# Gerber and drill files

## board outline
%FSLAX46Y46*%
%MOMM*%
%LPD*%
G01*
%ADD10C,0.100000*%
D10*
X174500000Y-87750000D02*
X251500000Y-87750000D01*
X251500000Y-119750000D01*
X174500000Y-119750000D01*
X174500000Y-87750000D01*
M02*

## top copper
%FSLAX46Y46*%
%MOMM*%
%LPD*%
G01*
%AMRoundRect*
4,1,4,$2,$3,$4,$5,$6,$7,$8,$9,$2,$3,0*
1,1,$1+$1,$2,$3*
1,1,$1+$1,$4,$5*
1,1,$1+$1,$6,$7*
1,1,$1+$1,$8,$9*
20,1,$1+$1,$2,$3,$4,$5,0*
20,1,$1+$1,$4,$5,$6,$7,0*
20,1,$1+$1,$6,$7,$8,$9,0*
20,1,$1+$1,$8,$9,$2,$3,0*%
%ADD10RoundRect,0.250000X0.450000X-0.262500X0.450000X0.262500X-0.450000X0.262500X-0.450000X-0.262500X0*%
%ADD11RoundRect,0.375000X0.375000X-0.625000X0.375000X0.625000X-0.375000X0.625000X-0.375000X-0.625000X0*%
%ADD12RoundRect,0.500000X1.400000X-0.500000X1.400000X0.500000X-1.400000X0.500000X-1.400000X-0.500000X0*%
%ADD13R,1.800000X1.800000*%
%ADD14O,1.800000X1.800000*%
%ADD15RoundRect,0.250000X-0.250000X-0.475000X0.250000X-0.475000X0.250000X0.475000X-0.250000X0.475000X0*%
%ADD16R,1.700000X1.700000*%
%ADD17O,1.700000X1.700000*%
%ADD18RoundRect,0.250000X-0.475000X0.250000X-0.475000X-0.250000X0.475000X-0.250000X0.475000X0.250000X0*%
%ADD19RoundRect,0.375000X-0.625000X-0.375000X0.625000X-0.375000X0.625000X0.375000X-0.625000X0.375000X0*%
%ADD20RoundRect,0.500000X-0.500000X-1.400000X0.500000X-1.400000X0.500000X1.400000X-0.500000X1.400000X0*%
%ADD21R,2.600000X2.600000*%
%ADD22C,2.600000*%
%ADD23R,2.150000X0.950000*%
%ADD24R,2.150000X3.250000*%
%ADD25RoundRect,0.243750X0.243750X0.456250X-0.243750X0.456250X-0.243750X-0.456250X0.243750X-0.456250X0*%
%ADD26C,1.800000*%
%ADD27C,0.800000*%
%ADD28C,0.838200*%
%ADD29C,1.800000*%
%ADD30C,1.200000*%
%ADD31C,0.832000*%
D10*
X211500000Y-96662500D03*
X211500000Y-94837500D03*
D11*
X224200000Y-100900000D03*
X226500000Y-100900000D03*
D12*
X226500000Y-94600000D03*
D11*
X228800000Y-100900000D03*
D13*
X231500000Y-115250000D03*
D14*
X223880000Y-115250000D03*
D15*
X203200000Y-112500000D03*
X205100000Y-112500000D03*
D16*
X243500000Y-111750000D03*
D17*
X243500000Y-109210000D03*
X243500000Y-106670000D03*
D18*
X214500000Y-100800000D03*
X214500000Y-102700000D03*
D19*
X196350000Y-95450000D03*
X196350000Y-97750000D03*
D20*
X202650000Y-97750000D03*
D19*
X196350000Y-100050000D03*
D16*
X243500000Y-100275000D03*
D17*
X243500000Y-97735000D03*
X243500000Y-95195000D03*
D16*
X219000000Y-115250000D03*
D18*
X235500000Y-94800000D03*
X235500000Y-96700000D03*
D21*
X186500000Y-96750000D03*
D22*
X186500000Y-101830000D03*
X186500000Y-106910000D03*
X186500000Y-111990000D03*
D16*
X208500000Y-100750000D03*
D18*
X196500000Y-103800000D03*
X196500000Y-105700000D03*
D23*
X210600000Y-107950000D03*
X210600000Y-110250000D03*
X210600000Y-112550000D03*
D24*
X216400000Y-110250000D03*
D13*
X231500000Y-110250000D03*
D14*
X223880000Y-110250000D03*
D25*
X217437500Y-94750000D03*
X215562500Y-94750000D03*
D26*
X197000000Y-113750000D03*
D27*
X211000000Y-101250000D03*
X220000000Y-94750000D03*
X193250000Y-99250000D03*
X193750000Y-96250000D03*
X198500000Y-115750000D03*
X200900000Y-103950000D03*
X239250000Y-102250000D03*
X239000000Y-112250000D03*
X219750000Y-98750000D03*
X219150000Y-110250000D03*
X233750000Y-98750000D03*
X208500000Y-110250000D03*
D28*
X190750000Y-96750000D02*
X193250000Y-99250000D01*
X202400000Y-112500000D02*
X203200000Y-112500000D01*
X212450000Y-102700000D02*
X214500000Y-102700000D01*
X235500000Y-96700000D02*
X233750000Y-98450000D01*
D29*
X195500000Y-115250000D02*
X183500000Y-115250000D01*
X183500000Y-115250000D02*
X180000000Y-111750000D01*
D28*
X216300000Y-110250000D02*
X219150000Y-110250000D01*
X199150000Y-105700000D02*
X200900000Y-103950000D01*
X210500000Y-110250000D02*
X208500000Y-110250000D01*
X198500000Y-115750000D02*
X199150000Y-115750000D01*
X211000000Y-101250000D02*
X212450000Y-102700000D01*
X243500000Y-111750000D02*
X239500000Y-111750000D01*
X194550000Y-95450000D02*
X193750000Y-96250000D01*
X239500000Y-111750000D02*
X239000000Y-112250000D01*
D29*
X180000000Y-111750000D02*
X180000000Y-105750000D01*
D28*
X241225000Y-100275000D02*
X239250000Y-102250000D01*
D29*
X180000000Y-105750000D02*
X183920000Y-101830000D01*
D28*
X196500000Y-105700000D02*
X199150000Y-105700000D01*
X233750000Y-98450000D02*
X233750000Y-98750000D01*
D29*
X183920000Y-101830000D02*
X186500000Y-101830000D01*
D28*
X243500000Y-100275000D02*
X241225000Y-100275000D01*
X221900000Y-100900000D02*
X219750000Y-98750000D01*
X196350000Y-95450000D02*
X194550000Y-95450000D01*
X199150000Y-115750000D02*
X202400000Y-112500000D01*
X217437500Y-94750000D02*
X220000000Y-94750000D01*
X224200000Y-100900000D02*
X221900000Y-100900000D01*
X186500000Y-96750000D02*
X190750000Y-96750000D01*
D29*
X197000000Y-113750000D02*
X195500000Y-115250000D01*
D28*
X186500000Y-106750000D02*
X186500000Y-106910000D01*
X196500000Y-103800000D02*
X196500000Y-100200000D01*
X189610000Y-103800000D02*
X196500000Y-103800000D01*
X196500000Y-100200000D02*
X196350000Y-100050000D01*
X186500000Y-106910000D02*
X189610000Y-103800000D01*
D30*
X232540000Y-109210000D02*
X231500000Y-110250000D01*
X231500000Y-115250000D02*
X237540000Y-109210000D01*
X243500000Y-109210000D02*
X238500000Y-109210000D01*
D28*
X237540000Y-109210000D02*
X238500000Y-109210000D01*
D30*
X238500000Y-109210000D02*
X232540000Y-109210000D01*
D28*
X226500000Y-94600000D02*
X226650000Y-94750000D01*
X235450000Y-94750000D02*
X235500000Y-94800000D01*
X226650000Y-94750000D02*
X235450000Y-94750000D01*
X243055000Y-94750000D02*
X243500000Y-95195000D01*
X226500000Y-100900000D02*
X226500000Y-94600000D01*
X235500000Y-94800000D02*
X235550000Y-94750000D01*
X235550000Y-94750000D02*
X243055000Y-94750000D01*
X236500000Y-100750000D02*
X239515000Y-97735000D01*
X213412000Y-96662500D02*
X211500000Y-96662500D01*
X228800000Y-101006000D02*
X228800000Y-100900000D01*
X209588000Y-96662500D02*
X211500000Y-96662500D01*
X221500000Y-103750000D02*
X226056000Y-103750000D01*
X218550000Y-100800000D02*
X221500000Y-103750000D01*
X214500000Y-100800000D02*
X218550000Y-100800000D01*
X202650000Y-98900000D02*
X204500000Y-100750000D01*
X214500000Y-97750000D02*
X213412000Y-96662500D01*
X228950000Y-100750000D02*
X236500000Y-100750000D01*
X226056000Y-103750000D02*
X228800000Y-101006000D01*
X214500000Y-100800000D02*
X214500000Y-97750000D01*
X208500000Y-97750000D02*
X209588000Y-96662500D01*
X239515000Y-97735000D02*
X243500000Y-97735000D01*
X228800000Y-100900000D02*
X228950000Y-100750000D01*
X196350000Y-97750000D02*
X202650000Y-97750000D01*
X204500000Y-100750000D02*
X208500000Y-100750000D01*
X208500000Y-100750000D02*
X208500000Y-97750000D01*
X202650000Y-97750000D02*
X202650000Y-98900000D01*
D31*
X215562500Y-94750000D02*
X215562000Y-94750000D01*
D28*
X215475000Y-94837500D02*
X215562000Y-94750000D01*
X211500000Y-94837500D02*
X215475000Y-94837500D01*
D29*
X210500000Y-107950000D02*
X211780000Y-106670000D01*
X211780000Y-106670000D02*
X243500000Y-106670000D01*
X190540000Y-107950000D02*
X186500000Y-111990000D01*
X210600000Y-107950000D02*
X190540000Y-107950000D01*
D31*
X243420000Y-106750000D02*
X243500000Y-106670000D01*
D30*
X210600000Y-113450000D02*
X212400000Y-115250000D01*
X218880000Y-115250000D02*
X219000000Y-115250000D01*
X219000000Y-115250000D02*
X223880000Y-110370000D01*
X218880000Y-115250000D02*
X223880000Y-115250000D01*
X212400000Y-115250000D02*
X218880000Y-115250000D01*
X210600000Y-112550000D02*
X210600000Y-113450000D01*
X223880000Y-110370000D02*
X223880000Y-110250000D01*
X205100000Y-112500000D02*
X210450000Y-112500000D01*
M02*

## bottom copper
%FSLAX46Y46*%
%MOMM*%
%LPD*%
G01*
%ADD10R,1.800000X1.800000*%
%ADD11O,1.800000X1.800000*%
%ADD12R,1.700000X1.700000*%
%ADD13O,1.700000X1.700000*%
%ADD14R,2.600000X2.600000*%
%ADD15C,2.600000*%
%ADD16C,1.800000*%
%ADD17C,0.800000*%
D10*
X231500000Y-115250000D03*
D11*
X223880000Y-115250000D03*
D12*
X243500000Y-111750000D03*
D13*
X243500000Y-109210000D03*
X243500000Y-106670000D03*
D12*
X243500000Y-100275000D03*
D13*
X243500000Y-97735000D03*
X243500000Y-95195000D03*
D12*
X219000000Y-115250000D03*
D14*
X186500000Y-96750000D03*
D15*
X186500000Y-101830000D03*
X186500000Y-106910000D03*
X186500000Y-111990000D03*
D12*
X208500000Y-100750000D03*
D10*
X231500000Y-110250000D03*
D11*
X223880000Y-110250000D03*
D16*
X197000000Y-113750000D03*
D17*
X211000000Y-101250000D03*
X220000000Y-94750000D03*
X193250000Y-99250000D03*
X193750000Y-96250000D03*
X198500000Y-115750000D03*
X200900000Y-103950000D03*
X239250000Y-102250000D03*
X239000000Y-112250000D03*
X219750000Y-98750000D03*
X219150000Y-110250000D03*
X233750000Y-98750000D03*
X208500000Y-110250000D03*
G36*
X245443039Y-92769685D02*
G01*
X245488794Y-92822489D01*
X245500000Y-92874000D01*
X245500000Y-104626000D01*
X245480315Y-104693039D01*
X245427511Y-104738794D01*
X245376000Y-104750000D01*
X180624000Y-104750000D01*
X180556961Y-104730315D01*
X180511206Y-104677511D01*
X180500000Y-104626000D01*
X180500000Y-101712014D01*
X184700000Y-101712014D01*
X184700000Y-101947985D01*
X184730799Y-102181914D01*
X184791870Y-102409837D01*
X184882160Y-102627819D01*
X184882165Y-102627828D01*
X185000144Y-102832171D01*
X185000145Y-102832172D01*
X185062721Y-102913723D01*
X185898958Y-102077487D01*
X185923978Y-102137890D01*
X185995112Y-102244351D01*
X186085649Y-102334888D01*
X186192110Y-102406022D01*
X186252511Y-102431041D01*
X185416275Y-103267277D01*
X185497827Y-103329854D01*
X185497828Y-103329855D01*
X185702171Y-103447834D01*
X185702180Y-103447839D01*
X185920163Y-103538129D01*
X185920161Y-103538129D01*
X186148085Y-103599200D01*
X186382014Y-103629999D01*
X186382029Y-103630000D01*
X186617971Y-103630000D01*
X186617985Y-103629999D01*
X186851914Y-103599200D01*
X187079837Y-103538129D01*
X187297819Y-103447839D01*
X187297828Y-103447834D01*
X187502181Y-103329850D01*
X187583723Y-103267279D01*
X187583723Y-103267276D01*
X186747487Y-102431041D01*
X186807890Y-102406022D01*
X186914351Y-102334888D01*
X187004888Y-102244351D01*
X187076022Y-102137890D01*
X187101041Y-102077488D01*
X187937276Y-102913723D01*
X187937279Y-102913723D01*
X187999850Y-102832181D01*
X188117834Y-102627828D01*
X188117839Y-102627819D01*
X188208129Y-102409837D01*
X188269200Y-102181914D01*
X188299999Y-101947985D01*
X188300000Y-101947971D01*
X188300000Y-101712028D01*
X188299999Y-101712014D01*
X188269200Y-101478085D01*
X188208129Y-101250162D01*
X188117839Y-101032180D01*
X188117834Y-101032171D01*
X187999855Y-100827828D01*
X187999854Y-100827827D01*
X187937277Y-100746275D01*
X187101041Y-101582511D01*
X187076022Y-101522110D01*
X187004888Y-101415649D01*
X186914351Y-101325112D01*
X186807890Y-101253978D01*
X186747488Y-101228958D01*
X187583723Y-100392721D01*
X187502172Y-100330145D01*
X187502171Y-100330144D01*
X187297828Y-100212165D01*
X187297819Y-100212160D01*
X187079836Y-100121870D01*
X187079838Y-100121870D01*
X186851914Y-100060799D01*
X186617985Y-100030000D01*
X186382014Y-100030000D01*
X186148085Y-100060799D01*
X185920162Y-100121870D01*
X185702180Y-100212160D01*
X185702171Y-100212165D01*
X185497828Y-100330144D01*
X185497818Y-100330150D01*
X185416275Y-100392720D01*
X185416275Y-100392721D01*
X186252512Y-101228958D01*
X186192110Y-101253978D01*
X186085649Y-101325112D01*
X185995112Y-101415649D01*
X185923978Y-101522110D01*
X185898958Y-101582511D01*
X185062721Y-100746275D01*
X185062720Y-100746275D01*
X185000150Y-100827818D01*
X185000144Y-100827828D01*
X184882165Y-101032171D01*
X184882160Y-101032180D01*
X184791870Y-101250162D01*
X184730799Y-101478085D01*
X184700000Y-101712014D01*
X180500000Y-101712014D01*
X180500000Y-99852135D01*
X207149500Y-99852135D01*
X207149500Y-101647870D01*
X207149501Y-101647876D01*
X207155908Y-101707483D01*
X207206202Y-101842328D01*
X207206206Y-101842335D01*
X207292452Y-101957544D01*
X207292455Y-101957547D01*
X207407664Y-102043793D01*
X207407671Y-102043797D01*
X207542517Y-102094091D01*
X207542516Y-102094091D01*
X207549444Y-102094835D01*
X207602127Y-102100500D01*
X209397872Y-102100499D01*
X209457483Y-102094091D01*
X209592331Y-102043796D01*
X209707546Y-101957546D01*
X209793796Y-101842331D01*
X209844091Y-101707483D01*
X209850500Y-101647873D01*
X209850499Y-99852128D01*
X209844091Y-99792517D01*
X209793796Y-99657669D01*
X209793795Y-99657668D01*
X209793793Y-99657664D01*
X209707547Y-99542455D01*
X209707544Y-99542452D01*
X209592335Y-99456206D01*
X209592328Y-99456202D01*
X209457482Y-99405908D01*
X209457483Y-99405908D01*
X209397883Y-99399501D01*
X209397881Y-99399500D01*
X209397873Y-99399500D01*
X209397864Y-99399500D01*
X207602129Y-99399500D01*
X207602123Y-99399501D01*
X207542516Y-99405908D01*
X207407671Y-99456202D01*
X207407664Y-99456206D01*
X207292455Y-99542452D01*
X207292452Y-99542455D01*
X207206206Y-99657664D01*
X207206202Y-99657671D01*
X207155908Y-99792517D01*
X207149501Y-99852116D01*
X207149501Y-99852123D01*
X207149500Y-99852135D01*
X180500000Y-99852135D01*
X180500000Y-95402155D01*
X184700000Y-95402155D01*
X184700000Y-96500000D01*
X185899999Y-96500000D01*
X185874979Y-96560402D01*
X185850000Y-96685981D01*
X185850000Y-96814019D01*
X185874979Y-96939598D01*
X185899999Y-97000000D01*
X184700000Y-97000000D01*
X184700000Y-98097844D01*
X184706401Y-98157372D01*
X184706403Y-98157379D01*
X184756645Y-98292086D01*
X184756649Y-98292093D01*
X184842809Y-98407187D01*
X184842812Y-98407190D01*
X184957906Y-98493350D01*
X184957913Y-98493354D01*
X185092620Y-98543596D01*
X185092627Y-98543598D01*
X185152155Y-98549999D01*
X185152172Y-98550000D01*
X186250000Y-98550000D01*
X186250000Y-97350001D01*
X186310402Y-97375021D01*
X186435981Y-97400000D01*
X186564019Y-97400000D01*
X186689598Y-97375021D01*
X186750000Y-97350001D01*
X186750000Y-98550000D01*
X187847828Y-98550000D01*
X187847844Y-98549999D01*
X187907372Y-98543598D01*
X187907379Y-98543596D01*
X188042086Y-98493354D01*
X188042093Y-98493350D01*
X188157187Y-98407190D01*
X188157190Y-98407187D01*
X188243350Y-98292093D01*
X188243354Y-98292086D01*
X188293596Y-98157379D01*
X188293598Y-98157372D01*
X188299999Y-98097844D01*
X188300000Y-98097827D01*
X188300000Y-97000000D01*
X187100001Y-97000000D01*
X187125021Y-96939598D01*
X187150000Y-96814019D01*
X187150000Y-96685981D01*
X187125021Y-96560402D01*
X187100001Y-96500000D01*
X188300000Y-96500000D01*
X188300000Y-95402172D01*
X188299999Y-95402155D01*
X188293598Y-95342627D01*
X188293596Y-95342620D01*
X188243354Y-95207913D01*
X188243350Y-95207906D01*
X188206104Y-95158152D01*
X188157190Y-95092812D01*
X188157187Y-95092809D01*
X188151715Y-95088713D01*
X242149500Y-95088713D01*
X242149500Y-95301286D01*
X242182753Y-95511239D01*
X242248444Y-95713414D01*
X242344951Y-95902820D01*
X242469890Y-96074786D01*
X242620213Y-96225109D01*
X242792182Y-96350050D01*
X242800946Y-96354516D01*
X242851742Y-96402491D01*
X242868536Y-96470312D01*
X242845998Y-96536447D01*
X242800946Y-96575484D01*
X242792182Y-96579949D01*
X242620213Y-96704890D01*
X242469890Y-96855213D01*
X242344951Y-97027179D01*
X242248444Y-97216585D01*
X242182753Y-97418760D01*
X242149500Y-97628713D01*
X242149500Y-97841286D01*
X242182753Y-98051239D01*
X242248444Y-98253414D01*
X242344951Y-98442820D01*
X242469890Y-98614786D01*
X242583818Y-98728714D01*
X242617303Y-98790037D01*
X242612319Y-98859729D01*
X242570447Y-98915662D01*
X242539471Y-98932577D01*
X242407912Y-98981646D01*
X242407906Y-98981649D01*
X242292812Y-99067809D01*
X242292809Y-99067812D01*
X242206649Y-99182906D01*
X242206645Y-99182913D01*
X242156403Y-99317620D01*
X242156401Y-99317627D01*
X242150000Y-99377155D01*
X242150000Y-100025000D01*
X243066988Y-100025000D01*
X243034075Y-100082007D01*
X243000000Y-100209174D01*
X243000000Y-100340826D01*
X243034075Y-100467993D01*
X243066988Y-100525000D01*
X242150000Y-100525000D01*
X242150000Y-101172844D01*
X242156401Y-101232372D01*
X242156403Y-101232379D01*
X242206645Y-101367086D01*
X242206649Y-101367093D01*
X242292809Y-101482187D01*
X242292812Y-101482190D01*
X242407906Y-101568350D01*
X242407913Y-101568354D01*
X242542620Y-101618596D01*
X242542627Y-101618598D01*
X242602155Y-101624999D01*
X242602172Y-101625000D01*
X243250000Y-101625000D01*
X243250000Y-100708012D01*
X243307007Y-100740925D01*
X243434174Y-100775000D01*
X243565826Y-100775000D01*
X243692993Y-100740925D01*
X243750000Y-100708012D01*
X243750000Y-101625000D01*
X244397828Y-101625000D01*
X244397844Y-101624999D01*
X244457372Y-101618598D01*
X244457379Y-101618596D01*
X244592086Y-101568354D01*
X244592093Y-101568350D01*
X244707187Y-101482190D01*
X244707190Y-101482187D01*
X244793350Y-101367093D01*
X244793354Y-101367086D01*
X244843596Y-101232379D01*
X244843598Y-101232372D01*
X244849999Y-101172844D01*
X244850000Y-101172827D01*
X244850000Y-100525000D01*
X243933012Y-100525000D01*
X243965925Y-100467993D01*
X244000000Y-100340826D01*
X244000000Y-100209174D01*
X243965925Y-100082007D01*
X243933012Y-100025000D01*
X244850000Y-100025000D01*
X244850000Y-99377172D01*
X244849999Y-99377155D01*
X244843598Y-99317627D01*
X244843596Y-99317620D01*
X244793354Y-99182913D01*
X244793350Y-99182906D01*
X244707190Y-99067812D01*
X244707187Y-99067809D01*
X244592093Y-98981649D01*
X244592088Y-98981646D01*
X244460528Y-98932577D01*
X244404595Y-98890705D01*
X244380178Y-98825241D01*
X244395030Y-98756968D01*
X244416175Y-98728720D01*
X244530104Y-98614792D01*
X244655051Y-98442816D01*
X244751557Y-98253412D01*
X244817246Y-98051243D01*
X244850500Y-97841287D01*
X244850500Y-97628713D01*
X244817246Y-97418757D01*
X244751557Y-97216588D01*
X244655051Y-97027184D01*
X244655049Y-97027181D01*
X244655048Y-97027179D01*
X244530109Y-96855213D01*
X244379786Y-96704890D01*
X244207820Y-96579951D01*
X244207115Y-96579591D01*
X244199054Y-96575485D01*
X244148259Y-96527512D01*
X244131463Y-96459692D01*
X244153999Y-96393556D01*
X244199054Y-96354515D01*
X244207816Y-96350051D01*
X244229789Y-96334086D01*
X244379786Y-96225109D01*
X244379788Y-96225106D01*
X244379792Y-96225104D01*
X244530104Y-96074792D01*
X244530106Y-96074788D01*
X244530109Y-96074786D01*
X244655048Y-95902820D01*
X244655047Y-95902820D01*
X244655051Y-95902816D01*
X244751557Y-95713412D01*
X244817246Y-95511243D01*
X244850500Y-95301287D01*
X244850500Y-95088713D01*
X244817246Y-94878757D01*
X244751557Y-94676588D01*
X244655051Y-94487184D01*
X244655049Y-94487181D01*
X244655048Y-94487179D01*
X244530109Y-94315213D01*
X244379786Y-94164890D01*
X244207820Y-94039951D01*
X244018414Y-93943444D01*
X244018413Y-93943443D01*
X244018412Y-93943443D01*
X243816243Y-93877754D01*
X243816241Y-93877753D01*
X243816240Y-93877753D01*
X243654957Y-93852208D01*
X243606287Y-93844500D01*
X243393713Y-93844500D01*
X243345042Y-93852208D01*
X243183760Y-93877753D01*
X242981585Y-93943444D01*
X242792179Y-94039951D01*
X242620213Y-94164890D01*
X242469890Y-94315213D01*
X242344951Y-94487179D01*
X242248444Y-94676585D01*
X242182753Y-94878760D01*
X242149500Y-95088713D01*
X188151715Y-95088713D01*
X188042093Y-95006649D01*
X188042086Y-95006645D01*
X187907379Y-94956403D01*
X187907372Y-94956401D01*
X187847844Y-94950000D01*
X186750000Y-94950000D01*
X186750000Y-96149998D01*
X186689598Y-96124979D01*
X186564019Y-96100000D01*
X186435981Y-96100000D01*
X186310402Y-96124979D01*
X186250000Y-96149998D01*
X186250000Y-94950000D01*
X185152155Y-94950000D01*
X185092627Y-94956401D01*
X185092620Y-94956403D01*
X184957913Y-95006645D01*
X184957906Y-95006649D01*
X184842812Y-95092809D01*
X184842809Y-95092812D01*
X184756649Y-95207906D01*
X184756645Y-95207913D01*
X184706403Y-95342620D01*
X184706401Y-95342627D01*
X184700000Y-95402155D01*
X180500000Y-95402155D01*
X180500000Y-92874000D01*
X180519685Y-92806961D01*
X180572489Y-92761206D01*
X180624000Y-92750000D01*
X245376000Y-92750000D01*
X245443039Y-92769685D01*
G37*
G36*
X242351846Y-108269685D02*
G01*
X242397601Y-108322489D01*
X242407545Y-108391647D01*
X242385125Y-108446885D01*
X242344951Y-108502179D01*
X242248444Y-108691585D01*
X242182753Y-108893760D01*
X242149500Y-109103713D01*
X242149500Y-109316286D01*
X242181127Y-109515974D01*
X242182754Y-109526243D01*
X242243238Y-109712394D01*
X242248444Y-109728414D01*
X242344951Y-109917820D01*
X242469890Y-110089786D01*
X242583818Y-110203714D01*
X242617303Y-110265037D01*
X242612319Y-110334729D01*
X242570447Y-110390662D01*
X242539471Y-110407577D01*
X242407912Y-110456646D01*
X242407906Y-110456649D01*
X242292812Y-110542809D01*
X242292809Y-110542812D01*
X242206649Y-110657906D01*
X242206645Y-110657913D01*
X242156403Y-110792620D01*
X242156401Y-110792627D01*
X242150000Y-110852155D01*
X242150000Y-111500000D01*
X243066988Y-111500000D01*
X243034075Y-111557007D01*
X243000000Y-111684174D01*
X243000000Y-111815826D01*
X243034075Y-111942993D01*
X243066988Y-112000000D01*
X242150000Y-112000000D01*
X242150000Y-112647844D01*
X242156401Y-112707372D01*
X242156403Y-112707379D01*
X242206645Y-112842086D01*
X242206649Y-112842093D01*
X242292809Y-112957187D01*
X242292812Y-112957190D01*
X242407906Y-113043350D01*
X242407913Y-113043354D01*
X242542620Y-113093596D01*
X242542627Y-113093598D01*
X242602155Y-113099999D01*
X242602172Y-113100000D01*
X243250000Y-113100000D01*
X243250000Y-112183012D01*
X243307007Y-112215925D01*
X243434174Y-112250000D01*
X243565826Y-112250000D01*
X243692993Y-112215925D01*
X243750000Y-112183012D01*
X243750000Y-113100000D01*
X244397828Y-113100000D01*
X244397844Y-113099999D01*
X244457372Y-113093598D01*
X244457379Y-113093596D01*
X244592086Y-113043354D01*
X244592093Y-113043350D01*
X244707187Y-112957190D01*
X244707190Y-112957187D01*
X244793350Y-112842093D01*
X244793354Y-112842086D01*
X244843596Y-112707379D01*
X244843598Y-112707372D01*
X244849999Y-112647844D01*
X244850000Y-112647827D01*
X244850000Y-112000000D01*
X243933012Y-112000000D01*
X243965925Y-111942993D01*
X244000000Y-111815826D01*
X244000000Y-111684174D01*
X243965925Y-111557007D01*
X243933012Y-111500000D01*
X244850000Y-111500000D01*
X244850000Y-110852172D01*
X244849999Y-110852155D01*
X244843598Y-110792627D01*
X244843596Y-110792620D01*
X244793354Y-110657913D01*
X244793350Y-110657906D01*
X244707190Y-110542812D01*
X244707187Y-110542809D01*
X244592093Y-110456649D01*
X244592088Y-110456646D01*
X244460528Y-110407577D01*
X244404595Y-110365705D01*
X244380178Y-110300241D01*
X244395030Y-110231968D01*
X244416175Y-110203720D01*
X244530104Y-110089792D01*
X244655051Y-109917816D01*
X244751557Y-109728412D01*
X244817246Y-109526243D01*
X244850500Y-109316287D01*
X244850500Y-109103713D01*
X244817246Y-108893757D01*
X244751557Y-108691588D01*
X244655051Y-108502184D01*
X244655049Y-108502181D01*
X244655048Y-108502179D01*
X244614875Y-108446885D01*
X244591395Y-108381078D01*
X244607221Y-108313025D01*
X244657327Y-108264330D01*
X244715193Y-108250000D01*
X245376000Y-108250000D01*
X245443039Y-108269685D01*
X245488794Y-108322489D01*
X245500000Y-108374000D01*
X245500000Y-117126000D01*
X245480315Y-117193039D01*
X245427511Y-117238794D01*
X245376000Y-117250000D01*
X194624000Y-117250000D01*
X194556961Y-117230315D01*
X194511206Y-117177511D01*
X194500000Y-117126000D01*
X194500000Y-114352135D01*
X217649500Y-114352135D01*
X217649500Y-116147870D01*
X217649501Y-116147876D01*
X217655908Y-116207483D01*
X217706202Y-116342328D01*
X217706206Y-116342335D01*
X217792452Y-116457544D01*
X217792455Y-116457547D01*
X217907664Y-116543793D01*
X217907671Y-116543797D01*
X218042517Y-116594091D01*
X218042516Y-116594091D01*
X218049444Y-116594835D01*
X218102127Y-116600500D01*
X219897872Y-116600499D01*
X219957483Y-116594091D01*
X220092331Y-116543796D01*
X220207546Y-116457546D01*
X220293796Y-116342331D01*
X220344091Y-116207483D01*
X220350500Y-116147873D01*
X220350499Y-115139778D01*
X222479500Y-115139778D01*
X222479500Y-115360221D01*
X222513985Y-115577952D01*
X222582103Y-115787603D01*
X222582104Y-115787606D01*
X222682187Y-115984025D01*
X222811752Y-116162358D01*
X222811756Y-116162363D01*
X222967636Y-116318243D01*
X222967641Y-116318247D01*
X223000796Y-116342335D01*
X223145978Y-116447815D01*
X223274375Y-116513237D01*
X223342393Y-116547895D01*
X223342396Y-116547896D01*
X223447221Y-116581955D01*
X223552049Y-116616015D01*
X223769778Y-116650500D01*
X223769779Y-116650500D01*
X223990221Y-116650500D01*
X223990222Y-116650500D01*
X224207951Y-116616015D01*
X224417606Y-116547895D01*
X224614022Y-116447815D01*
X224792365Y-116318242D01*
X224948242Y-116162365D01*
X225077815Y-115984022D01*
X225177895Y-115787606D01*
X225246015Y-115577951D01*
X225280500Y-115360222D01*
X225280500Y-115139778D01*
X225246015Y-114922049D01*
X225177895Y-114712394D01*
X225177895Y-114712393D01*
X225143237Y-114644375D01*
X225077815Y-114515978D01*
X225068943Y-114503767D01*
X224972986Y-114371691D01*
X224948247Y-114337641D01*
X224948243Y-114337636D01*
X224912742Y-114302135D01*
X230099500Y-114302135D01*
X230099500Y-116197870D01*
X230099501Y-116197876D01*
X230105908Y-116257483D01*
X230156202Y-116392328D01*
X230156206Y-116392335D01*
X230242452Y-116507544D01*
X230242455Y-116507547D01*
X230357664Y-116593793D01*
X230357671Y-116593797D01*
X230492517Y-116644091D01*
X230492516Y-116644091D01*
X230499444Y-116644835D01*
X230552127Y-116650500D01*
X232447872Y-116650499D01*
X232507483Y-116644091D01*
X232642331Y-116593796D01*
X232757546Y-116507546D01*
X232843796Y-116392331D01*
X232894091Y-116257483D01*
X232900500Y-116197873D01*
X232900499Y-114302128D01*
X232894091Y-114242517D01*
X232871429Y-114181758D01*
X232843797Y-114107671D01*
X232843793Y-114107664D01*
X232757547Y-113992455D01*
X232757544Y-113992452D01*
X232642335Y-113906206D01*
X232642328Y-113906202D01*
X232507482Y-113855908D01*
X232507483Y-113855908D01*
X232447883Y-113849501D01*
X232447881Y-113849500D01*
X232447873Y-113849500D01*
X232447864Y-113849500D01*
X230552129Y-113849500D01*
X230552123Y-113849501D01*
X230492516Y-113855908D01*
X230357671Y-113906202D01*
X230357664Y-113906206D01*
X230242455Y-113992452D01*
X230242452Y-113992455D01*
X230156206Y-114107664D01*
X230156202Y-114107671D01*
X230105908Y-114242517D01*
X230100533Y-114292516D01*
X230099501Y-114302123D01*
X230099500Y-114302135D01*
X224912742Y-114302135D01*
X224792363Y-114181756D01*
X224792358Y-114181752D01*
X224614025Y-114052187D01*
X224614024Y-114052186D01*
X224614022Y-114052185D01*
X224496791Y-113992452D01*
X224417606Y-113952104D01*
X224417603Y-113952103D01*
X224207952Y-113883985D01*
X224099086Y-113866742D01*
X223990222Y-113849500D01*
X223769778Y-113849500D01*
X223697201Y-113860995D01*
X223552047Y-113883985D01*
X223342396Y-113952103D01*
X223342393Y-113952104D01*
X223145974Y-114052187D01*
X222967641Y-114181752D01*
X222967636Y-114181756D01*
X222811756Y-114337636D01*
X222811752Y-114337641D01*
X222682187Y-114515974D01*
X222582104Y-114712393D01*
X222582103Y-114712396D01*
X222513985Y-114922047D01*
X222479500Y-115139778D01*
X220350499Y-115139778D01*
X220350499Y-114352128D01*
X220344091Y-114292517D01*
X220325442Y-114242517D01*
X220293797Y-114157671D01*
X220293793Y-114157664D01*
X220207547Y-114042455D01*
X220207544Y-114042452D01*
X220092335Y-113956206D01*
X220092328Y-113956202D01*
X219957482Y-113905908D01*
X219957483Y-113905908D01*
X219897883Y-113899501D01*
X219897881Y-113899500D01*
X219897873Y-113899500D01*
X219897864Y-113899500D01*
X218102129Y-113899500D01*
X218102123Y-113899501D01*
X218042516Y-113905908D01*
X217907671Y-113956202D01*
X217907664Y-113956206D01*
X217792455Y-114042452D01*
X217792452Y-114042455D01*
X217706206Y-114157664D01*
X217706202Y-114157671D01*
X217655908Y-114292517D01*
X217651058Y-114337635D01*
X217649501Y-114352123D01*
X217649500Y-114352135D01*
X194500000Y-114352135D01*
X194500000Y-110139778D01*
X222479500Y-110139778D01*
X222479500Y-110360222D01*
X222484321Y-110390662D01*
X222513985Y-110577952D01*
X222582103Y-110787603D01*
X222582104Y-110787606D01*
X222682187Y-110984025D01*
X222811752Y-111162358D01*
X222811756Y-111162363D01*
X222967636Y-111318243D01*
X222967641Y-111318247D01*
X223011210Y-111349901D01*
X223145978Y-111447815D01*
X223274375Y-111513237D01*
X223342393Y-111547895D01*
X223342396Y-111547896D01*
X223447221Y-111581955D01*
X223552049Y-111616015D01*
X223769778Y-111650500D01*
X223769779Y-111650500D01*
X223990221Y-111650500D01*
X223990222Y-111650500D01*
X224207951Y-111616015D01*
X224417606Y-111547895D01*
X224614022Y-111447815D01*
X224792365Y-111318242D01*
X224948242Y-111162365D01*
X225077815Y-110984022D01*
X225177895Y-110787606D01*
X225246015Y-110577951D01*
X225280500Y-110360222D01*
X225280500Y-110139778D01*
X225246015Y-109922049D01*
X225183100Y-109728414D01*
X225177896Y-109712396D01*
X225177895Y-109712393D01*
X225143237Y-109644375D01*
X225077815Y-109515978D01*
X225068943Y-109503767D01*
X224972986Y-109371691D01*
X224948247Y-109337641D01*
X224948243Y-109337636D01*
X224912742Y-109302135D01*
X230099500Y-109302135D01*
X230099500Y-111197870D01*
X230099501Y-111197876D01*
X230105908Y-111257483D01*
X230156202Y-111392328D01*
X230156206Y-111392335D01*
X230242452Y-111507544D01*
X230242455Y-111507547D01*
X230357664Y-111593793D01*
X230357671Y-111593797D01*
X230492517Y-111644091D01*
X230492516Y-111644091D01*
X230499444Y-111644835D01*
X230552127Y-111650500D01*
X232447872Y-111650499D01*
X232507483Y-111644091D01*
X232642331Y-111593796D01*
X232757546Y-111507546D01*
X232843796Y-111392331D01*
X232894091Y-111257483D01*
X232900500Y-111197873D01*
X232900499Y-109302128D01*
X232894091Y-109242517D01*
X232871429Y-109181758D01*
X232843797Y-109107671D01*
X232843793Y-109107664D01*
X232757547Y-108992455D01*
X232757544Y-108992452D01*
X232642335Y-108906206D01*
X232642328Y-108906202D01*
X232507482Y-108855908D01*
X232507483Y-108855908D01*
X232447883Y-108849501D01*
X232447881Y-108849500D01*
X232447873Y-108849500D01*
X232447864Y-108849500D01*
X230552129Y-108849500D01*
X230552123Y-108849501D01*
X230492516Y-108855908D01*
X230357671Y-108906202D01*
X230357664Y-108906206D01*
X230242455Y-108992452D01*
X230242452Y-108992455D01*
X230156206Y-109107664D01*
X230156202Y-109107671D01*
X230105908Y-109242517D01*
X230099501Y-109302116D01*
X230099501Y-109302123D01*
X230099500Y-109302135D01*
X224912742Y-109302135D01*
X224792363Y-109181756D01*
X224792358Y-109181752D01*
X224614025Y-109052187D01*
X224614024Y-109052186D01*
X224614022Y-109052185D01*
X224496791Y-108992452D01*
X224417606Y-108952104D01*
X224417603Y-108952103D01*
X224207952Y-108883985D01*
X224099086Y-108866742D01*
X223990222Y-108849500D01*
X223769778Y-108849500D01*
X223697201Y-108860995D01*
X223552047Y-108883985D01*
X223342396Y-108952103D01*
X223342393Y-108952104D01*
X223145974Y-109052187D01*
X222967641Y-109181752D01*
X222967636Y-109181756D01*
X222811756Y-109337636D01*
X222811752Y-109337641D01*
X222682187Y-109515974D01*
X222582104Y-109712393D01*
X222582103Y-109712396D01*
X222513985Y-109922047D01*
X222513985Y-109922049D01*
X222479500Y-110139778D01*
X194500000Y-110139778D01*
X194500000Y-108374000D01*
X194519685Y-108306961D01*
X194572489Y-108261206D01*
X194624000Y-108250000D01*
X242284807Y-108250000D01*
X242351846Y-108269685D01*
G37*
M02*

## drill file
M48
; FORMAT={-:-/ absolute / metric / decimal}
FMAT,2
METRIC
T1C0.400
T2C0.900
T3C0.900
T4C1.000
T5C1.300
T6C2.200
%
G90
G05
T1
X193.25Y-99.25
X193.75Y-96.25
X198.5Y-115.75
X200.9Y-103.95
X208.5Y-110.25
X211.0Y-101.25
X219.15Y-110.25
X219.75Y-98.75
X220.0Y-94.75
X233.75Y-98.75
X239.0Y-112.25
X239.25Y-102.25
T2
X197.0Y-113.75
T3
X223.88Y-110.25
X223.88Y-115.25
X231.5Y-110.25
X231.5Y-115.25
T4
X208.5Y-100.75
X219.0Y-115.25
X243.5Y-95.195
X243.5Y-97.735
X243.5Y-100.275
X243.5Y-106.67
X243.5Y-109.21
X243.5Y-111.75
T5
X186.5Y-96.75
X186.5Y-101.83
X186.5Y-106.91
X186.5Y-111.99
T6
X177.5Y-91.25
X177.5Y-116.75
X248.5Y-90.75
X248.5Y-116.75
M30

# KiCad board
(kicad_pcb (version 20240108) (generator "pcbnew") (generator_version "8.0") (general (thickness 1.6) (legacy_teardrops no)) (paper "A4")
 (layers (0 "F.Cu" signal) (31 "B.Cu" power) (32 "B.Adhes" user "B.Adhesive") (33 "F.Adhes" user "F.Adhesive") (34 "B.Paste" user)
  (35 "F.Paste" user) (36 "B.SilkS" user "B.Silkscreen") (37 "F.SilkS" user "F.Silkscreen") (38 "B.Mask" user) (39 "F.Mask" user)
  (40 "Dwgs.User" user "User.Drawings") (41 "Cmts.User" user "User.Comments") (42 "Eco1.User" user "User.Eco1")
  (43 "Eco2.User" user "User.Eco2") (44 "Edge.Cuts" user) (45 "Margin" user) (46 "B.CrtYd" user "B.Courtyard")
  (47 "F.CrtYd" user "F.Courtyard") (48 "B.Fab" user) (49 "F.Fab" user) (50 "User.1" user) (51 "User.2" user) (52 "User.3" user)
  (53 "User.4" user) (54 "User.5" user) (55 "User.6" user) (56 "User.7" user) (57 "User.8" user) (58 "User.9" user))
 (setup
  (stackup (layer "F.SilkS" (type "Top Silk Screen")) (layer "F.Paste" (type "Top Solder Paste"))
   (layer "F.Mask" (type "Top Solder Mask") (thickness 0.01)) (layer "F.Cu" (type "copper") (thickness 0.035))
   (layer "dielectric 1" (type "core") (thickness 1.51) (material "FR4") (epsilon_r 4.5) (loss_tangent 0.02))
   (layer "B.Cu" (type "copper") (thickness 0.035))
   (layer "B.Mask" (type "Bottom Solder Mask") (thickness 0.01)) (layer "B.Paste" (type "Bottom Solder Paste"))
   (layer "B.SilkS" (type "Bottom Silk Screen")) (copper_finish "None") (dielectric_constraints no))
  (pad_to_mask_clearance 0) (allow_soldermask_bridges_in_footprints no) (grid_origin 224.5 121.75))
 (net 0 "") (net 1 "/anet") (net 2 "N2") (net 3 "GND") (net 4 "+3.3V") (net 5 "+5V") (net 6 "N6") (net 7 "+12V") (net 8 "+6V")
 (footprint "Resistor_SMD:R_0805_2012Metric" (layer "F.Cu") (at 211.5 95.75 90)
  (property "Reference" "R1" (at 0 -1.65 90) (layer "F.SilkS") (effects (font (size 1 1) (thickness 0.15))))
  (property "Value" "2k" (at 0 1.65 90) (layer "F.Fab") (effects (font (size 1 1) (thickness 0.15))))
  (pad "1" smd roundrect (at -0.9125 0 90) (size 1.025 1.4) (layers "F.Cu" "F.Paste" "F.Mask") (roundrect_rratio 0.243902) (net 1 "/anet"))
  (pad "2" smd roundrect (at 0.9125 0 90) (size 1.025 1.4) (layers "F.Cu" "F.Paste" "F.Mask") (roundrect_rratio 0.243902) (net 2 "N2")))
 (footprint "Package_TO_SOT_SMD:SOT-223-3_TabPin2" (layer "F.Cu") (at 226.5 97.75 90)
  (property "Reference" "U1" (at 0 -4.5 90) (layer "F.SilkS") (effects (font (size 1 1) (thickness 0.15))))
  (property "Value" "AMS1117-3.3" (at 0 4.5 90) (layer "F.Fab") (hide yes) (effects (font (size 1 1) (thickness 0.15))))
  (pad "1" smd roundrect (at -3.15 -2.3 90) (size 2 1.5) (layers "F.Cu" "F.Paste" "F.Mask") (roundrect_rratio 0.25) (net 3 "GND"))
  (pad "2" smd roundrect (at -3.15 0 90) (size 2 1.5) (layers "F.Cu" "F.Paste" "F.Mask") (roundrect_rratio 0.25) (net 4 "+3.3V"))
  (pad "2" smd roundrect (at 3.15 0 90) (size 2 3.8) (layers "F.Cu" "F.Paste" "F.Mask") (roundrect_rratio 0.25) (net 4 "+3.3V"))
  (pad "3" smd roundrect (at -3.15 2.3 90) (size 2 1.5) (layers "F.Cu" "F.Paste" "F.Mask") (roundrect_rratio 0.25) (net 1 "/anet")))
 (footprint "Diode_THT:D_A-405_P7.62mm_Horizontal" (layer "F.Cu") (at 231.5 115.25 180)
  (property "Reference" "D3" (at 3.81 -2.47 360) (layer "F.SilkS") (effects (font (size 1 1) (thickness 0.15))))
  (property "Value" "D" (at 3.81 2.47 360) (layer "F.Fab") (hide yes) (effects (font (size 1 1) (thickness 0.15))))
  (pad "1" thru_hole rect (at 0 0 180) (size 1.8 1.8) (drill 0.9) (layers "*.Cu" "*.Mask") (remove_unused_layers no) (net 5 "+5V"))
  (pad "2" thru_hole oval (at 7.62 0 180) (size 1.8 1.8) (drill 0.9) (layers "*.Cu" "*.Mask") (remove_unused_layers no) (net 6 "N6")))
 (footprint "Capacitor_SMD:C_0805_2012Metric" (layer "F.Cu") (at 204.15 112.5)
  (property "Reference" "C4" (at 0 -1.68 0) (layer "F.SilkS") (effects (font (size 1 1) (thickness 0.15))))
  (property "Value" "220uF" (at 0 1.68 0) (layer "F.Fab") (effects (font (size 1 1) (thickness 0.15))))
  (pad "1" smd roundrect (at -0.95 0) (size 1 1.45) (layers "F.Cu" "F.Paste" "F.Mask") (roundrect_rratio 0.25) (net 3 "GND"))
  (pad "2" smd roundrect (at 0.95 0) (size 1 1.45) (layers "F.Cu" "F.Paste" "F.Mask") (roundrect_rratio 0.25) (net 6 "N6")))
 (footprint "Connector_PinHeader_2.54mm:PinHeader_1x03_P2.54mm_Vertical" (layer "F.Cu") (at 243.5 111.75 180)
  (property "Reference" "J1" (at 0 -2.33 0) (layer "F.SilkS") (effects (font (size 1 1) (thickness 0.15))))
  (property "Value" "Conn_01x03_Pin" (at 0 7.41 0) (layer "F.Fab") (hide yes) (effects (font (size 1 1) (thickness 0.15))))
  (pad "1" thru_hole rect (at 0 0 180) (size 1.7 1.7) (drill 1) (layers "*.Cu" "*.Mask") (remove_unused_layers no) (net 3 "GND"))
  (pad "2" thru_hole oval (at 0 2.54 180) (size 1.7 1.7) (drill 1) (layers "*.Cu" "*.Mask") (remove_unused_layers no) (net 5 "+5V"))
  (pad "3" thru_hole oval (at 0 5.08 180) (size 1.7 1.7) (drill 1) (layers "*.Cu" "*.Mask") (remove_unused_layers no) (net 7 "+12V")))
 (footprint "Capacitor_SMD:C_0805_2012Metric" (layer "F.Cu") (at 214.5 101.75 -90)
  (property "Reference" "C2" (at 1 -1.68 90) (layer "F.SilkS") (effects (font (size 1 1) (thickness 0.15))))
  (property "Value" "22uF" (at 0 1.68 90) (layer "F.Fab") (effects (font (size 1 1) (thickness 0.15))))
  (pad "1" smd roundrect (at -0.95 0 270) (size 1 1.45) (layers "F.Cu" "F.Paste" "F.Mask") (roundrect_rratio 0.25) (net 1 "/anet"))
  (pad "2" smd roundrect (at 0.95 0 270) (size 1 1.45) (layers "F.Cu" "F.Paste" "F.Mask") (roundrect_rratio 0.25) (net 3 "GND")))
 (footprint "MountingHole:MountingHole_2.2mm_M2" (layer "F.Cu") (at 177.5 116.75)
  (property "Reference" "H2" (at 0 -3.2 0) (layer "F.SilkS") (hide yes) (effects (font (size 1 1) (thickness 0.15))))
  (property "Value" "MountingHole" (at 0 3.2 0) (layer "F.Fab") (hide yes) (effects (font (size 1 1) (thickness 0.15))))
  (pad "" np_thru_hole circle (at 0 0) (size 2.2 2.2) (drill 2.2) (layers "*.Cu" "*.Mask")))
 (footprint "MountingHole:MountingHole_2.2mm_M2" (layer "F.Cu") (at 177.5 91.25)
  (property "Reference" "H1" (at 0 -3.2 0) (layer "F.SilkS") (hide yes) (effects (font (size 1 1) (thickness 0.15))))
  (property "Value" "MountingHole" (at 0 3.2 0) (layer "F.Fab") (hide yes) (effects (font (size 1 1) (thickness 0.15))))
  (pad "" np_thru_hole circle (at 0 0) (size 2.2 2.2) (drill 2.2) (layers "*.Cu" "*.Mask")))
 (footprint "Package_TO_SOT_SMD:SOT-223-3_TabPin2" (layer "F.Cu") (at 199.5 97.75)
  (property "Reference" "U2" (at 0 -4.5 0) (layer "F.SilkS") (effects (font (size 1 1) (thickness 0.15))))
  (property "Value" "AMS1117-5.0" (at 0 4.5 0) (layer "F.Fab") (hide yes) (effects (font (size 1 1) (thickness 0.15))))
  (pad "1" smd roundrect (at -3.15 -2.3) (size 2 1.5) (layers "F.Cu" "F.Paste" "F.Mask") (roundrect_rratio 0.25) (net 3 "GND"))
  (pad "2" smd roundrect (at -3.15 0) (size 2 1.5) (layers "F.Cu" "F.Paste" "F.Mask") (roundrect_rratio 0.25) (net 1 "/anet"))
  (pad "2" smd roundrect (at 3.15 0) (size 2 3.8) (layers "F.Cu" "F.Paste" "F.Mask") (roundrect_rratio 0.25) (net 1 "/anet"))
  (pad "3" smd roundrect (at -3.15 2.3) (size 2 1.5) (layers "F.Cu" "F.Paste" "F.Mask") (roundrect_rratio 0.25) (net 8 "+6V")))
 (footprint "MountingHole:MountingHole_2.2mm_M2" (layer "F.Cu") (at 248.5 90.75)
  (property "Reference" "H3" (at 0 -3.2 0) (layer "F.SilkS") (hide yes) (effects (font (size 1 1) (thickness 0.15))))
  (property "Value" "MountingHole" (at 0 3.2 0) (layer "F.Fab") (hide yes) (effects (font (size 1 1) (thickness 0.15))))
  (pad "" np_thru_hole circle (at 0 0) (size 2.2 2.2) (drill 2.2) (layers "*.Cu" "*.Mask")))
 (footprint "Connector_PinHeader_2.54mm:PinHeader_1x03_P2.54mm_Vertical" (layer "F.Cu") (at 243.5 100.275 180)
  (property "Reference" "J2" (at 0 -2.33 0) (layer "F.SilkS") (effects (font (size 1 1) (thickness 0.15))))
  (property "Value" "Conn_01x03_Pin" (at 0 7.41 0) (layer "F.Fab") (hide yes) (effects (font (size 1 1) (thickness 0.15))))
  (pad "1" thru_hole rect (at 0 0 180) (size 1.7 1.7) (drill 1) (layers "*.Cu" "*.Mask") (remove_unused_layers no) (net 3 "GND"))
  (pad "2" thru_hole oval (at 0 2.54 180) (size 1.7 1.7) (drill 1) (layers "*.Cu" "*.Mask") (remove_unused_layers no) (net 1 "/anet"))
  (pad "3" thru_hole oval (at 0 5.08 180) (size 1.7 1.7) (drill 1) (layers "*.Cu" "*.Mask") (remove_unused_layers no) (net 4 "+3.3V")))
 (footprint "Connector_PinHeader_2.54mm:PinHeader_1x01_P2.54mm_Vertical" (layer "F.Cu") (at 219 115.25)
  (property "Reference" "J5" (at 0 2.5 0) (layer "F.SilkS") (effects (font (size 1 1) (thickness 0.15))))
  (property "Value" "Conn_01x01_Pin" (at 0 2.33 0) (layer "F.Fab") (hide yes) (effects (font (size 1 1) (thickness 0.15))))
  (pad "1" thru_hole rect (at 0 0) (size 1.7 1.7) (drill 1) (layers "*.Cu" "*.Mask") (remove_unused_layers no) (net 6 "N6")))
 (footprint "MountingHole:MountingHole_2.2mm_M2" (layer "F.Cu") (at 248.5 116.75)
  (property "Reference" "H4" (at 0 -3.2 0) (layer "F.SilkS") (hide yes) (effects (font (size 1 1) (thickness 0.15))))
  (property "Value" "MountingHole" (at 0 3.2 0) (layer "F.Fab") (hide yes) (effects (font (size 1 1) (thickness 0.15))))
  (pad "" np_thru_hole circle (at 0 0) (size 2.2 2.2) (drill 2.2) (layers "*.Cu" "*.Mask")))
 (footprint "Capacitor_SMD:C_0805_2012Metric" (layer "F.Cu") (at 235.5 95.75 -90)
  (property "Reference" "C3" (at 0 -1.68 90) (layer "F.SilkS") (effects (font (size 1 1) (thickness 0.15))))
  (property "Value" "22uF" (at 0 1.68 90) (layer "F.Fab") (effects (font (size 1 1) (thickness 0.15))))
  (pad "1" smd roundrect (at -0.95 0 270) (size 1 1.45) (layers "F.Cu" "F.Paste" "F.Mask") (roundrect_rratio 0.25) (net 4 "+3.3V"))
  (pad "2" smd roundrect (at 0.95 0 270) (size 1 1.45) (layers "F.Cu" "F.Paste" "F.Mask") (roundrect_rratio 0.25) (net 3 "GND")))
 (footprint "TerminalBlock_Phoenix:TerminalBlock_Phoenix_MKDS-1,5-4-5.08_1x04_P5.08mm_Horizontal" (layer "F.Cu") (at 186.5 96.75 -90)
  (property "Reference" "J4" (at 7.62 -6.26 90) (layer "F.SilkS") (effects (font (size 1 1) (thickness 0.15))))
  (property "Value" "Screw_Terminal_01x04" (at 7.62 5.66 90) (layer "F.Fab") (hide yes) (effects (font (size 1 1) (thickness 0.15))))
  (pad "1" thru_hole rect (at 0 0 270) (size 2.6 2.6) (drill 1.3) (layers "*.Cu" "*.Mask") (remove_unused_layers no) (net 3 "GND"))
  (pad "2" thru_hole circle (at 5.08 0 270) (size 2.6 2.6) (drill 1.3) (layers "*.Cu" "*.Mask") (remove_unused_layers no) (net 3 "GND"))
  (pad "3" thru_hole circle (at 10.16 0 270) (size 2.6 2.6) (drill 1.3) (layers "*.Cu" "*.Mask") (remove_unused_layers no) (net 8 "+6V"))
  (pad "4" thru_hole circle (at 15.24 0 270) (size 2.6 2.6) (drill 1.3) (layers "*.Cu" "*.Mask") (remove_unused_layers no) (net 7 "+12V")))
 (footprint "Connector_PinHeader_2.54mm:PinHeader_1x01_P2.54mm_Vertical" (layer "F.Cu") (at 208.5 100.75)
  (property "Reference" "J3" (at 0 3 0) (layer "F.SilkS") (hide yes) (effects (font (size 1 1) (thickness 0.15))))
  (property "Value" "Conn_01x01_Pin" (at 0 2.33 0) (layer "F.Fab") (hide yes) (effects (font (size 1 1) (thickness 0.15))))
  (pad "1" thru_hole rect (at 0 0) (size 1.7 1.7) (drill 1) (layers "*.Cu" "*.Mask") (remove_unused_layers no) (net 1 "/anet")))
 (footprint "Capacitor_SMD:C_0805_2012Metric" (layer "F.Cu") (at 196.5 104.75 -90)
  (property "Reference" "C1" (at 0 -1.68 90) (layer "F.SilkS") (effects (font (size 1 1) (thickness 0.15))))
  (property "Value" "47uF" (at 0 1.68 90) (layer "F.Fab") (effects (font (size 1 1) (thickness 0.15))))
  (pad "1" smd roundrect (at -0.95 0 270) (size 1 1.45) (layers "F.Cu" "F.Paste" "F.Mask") (roundrect_rratio 0.25) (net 8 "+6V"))
  (pad "2" smd roundrect (at 0.95 0 270) (size 1 1.45) (layers "F.Cu" "F.Paste" "F.Mask") (roundrect_rratio 0.25) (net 3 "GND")))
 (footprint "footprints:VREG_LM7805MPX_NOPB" (layer "F.Cu") (at 213.5 110.25)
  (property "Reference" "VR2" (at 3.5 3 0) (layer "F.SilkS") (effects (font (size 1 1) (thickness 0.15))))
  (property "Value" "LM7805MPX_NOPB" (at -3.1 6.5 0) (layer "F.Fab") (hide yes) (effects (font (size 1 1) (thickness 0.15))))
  (pad "1" smd rect (at -2.9 -2.3) (size 2.15 0.95) (layers "F.Cu" "F.Paste" "F.Mask") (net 7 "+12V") (solder_mask_margin 0.102))
  (pad "2" smd rect (at -2.9 0) (size 2.15 0.95) (layers "F.Cu" "F.Paste" "F.Mask") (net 3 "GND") (solder_mask_margin 0.102))
  (pad "3" smd rect (at -2.9 2.3) (size 2.15 0.95) (layers "F.Cu" "F.Paste" "F.Mask") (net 6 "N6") (solder_mask_margin 0.102))
  (pad "4" smd rect (at 2.9 0) (size 2.15 3.25) (layers "F.Cu" "F.Paste" "F.Mask") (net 3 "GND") (solder_mask_margin 0.102)))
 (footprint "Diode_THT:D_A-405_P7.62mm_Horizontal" (layer "F.Cu") (at 231.5 110.25 180)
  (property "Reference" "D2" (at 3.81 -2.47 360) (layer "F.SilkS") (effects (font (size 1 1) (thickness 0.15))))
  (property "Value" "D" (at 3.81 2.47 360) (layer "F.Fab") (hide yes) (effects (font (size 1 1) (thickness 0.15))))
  (pad "1" thru_hole rect (at 0 0 180) (size 1.8 1.8) (drill 0.9) (layers "*.Cu" "*.Mask") (remove_unused_layers no) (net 5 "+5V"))
  (pad "2" thru_hole oval (at 7.62 0 180) (size 1.8 1.8) (drill 0.9) (layers "*.Cu" "*.Mask") (remove_unused_layers no) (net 6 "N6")))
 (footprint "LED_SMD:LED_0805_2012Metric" (layer "F.Cu") (at 216.5 94.75 180)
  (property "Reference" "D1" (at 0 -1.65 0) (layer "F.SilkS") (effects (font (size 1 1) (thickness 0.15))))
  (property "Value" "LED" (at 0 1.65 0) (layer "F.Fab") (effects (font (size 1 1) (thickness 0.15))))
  (pad "1" smd roundrect (at -0.9375 0 180) (size 0.975 1.4) (layers "F.Cu" "F.Paste" "F.Mask") (roundrect_rratio 0.25) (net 3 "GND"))
  (pad "2" smd roundrect (at 0.9375 0 180) (size 0.975 1.4) (layers "F.Cu" "F.Paste" "F.Mask") (roundrect_rratio 0.25) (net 2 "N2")))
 (gr_rect (start 174.5 87.75) (end 251.5 119.75) (stroke (width 0.1) (type default)) (fill none) (layer "Edge.Cuts"))
 (segment (start 190.75 96.75) (end 193.25 99.25) (width 0.8382) (layer "F.Cu") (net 3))
 (segment (start 202.4 112.5) (end 203.2 112.5) (width 0.8382) (layer "F.Cu") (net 3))
 (segment (start 212.45 102.7) (end 214.5 102.7) (width 0.8382) (layer "F.Cu") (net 3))
 (segment (start 235.5 96.7) (end 233.75 98.45) (width 0.8382) (layer "F.Cu") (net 3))
 (segment (start 195.5 115.25) (end 183.5 115.25) (width 1.8) (layer "F.Cu") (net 3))
 (segment (start 183.5 115.25) (end 180 111.75) (width 1.8) (layer "F.Cu") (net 3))
 (segment (start 216.3 110.25) (end 219.15 110.25) (width 0.8382) (layer "F.Cu") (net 3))
 (segment (start 199.15 105.7) (end 200.9 103.95) (width 0.8382) (layer "F.Cu") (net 3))
 (segment (start 210.5 110.25) (end 208.5 110.25) (width 0.8382) (layer "F.Cu") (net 3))
 (segment (start 198.5 115.75) (end 199.15 115.75) (width 0.8382) (layer "F.Cu") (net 3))
 (segment (start 211 101.25) (end 212.45 102.7) (width 0.8382) (layer "F.Cu") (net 3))
 (segment (start 243.5 111.75) (end 239.5 111.75) (width 0.8382) (layer "F.Cu") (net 3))
 (segment (start 194.55 95.45) (end 193.75 96.25) (width 0.8382) (layer "F.Cu") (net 3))
 (segment (start 239.5 111.75) (end 239 112.25) (width 0.8382) (layer "F.Cu") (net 3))
 (segment (start 180 111.75) (end 180 105.75) (width 1.8) (layer "F.Cu") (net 3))
 (segment (start 241.225 100.275) (end 239.25 102.25) (width 0.8382) (layer "F.Cu") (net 3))
 (segment (start 180 105.75) (end 183.92 101.83) (width 1.8) (layer "F.Cu") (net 3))
 (segment (start 196.5 105.7) (end 199.15 105.7) (width 0.8382) (layer "F.Cu") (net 3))
 (segment (start 233.75 98.45) (end 233.75 98.75) (width 0.8382) (layer "F.Cu") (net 3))
 (segment (start 183.92 101.83) (end 186.5 101.83) (width 1.8) (layer "F.Cu") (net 3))
 (segment (start 243.5 100.275) (end 241.225 100.275) (width 0.8382) (layer "F.Cu") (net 3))
 (segment (start 221.9 100.9) (end 219.75 98.75) (width 0.8382) (layer "F.Cu") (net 3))
 (segment (start 196.35 95.45) (end 194.55 95.45) (width 0.8382) (layer "F.Cu") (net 3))
 (segment (start 199.15 115.75) (end 202.4 112.5) (width 0.8382) (layer "F.Cu") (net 3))
 (segment (start 217.4375 94.75) (end 220 94.75) (width 0.8382) (layer "F.Cu") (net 3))
 (segment (start 224.2 100.9) (end 221.9 100.9) (width 0.8382) (layer "F.Cu") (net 3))
 (segment (start 186.5 96.75) (end 190.75 96.75) (width 0.8382) (layer "F.Cu") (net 3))
 (segment (start 197 113.75) (end 195.5 115.25) (width 1.8) (layer "F.Cu") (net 3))
 (via (at 197 113.75) (size 1.8) (drill 0.9) (layers "F.Cu" "B.Cu") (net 3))
 (via (at 211 101.25) (size 0.8) (drill 0.4) (layers "F.Cu" "B.Cu") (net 3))
 (via (at 220 94.75) (size 0.8) (drill 0.4) (layers "F.Cu" "B.Cu") (free yes) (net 3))
 (via (at 193.25 99.25) (size 0.8) (drill 0.4) (layers "F.Cu" "B.Cu") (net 3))
 (via (at 193.75 96.25) (size 0.8) (drill 0.4) (layers "F.Cu" "B.Cu") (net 3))
 (via (at 198.5 115.75) (size 0.8) (drill 0.4) (layers "F.Cu" "B.Cu") (free yes) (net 3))
 (via (at 200.9 103.95) (size 0.8) (drill 0.4) (layers "F.Cu" "B.Cu") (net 3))
 (via (at 239.25 102.25) (size 0.8) (drill 0.4) (layers "F.Cu" "B.Cu") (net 3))
 (via (at 239 112.25) (size 0.8) (drill 0.4) (layers "F.Cu" "B.Cu") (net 3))
 (via (at 219.75 98.75) (size 0.8) (drill 0.4) (layers "F.Cu" "B.Cu") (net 3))
 (via (at 219.15 110.25) (size 0.8) (drill 0.4) (layers "F.Cu" "B.Cu") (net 3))
 (via (at 233.75 98.75) (size 0.8) (drill 0.4) (layers "F.Cu" "B.Cu") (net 3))
 (via (at 208.5 110.25) (size 0.8) (drill 0.4) (layers "F.Cu" "B.Cu") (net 3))
 (segment (start 186.5 106.75) (end 186.5 106.91) (width 0.8382) (layer "F.Cu") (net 8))
 (segment (start 196.5 103.8) (end 196.5 100.2) (width 0.8382) (layer "F.Cu") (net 8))
 (segment (start 189.61 103.8) (end 196.5 103.8) (width 0.8382) (layer "F.Cu") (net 8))
 (segment (start 196.5 100.2) (end 196.35 100.05) (width 0.8382) (layer "F.Cu") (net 8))
 (segment (start 186.5 106.91) (end 189.61 103.8) (width 0.8382) (layer "F.Cu") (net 8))
 (segment (start 232.54 109.21) (end 231.5 110.25) (width 1.2) (layer "F.Cu") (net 5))
 (segment (start 231.5 115.25) (end 237.54 109.21) (width 1.2) (layer "F.Cu") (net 5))
 (segment (start 243.5 109.21) (end 238.5 109.21) (width 1.2) (layer "F.Cu") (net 5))
 (segment (start 237.54 109.21) (end 238.5 109.21) (width 0.8382) (layer "F.Cu") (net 5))
 (segment (start 238.5 109.21) (end 232.54 109.21) (width 1.2) (layer "F.Cu") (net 5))
 (segment (start 226.5 94.6) (end 226.65 94.75) (width 0.8382) (layer "F.Cu") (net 4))
 (segment (start 235.45 94.75) (end 235.5 94.8) (width 0.8382) (layer "F.Cu") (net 4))
 (segment (start 226.65 94.75) (end 235.45 94.75) (width 0.8382) (layer "F.Cu") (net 4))
 (segment (start 243.055 94.75) (end 243.5 95.195) (width 0.8382) (layer "F.Cu") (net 4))
 (segment (start 226.5 100.9) (end 226.5 94.6) (width 0.8382) (layer "F.Cu") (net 4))
 (segment (start 235.5 94.8) (end 235.55 94.75) (width 0.8382) (layer "F.Cu") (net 4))
 (segment (start 235.55 94.75) (end 243.055 94.75) (width 0.8382) (layer "F.Cu") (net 4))
 (segment (start 236.5 100.75) (end 239.515 97.735) (width 0.8382) (layer "F.Cu") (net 1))
 (segment (start 213.412 96.6625) (end 211.5 96.6625) (width 0.8382) (layer "F.Cu") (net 1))
 (segment (start 228.8 101.006) (end 228.8 100.9) (width 0.8382) (layer "F.Cu") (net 1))
 (segment (start 209.588 96.6625) (end 211.5 96.6625) (width 0.8382) (layer "F.Cu") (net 1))
 (segment (start 221.5 103.75) (end 226.056 103.75) (width 0.8382) (layer "F.Cu") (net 1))
 (segment (start 218.55 100.8) (end 221.5 103.75) (width 0.8382) (layer "F.Cu") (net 1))
 (segment (start 214.5 100.8) (end 218.55 100.8) (width 0.8382) (layer "F.Cu") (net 1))
 (segment (start 202.65 98.9) (end 204.5 100.75) (width 0.8382) (layer "F.Cu") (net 1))
 (segment (start 214.5 97.75) (end 213.412 96.6625) (width 0.8382) (layer "F.Cu") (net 1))
 (segment (start 228.95 100.75) (end 236.5 100.75) (width 0.8382) (layer "F.Cu") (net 1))
 (segment (start 226.056 103.75) (end 228.8 101.006) (width 0.8382) (layer "F.Cu") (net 1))
 (segment (start 214.5 100.8) (end 214.5 97.75) (width 0.8382) (layer "F.Cu") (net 1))
 (segment (start 208.5 97.75) (end 209.588 96.6625) (width 0.8382) (layer "F.Cu") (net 1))
 (segment (start 239.515 97.735) (end 243.5 97.735) (width 0.8382) (layer "F.Cu") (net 1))
 (segment (start 228.8 100.9) (end 228.95 100.75) (width 0.8382) (layer "F.Cu") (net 1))
 (segment (start 196.35 97.75) (end 202.65 97.75) (width 0.8382) (layer "F.Cu") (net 1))
 (segment (start 204.5 100.75) (end 208.5 100.75) (width 0.8382) (layer "F.Cu") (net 1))
 (segment (start 208.5 100.75) (end 208.5 97.75) (width 0.8382) (layer "F.Cu") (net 1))
 (segment (start 202.65 97.75) (end 202.65 98.9) (width 0.8382) (layer "F.Cu") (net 1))
 (segment (start 215.5625 94.75) (end 215.562 94.75) (width 0.832) (layer "F.Cu") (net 2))
 (segment (start 215.475 94.8375) (end 215.562 94.75) (width 0.8382) (layer "F.Cu") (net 2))
 (segment (start 211.5 94.8375) (end 215.475 94.8375) (width 0.8382) (layer "F.Cu") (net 2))
 (segment (start 210.5 107.95) (end 211.78 106.67) (width 1.8) (layer "F.Cu") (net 7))
 (segment (start 211.78 106.67) (end 243.5 106.67) (width 1.8) (layer "F.Cu") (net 7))
 (segment (start 190.54 107.95) (end 186.5 111.99) (width 1.8) (layer "F.Cu") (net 7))
 (segment (start 210.6 107.95) (end 190.54 107.95) (width 1.8) (layer "F.Cu") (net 7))
 (segment (start 243.42 106.75) (end 243.5 106.67) (width 0.832) (layer "F.Cu") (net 7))
 (segment (start 210.6 113.45) (end 212.4 115.25) (width 1.2) (layer "F.Cu") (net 6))
 (segment (start 218.88 115.25) (end 219 115.25) (width 1.2) (layer "F.Cu") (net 6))
 (segment (start 219 115.25) (end 223.88 110.37) (width 1.2) (layer "F.Cu") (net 6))
 (segment (start 218.88 115.25) (end 223.88 115.25) (width 1.2) (layer "F.Cu") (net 6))
 (segment (start 212.4 115.25) (end 218.88 115.25) (width 1.2) (layer "F.Cu") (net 6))
 (segment (start 210.6 112.55) (end 210.6 113.45) (width 1.2) (layer "F.Cu") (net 6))
 (segment (start 223.88 110.37) (end 223.88 110.25) (width 1.2) (layer "F.Cu") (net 6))
 (segment (start 205.1 112.5) (end 210.45 112.5) (width 1.2) (layer "F.Cu") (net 6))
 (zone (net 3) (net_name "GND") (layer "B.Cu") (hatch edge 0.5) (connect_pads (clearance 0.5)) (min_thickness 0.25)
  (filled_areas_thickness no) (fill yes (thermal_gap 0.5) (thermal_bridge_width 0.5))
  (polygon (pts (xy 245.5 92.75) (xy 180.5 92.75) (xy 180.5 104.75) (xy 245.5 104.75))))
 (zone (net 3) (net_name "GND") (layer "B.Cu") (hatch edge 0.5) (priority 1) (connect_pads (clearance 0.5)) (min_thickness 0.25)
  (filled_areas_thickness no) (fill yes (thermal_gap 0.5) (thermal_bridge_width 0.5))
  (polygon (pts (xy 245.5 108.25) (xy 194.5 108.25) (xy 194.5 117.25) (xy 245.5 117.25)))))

